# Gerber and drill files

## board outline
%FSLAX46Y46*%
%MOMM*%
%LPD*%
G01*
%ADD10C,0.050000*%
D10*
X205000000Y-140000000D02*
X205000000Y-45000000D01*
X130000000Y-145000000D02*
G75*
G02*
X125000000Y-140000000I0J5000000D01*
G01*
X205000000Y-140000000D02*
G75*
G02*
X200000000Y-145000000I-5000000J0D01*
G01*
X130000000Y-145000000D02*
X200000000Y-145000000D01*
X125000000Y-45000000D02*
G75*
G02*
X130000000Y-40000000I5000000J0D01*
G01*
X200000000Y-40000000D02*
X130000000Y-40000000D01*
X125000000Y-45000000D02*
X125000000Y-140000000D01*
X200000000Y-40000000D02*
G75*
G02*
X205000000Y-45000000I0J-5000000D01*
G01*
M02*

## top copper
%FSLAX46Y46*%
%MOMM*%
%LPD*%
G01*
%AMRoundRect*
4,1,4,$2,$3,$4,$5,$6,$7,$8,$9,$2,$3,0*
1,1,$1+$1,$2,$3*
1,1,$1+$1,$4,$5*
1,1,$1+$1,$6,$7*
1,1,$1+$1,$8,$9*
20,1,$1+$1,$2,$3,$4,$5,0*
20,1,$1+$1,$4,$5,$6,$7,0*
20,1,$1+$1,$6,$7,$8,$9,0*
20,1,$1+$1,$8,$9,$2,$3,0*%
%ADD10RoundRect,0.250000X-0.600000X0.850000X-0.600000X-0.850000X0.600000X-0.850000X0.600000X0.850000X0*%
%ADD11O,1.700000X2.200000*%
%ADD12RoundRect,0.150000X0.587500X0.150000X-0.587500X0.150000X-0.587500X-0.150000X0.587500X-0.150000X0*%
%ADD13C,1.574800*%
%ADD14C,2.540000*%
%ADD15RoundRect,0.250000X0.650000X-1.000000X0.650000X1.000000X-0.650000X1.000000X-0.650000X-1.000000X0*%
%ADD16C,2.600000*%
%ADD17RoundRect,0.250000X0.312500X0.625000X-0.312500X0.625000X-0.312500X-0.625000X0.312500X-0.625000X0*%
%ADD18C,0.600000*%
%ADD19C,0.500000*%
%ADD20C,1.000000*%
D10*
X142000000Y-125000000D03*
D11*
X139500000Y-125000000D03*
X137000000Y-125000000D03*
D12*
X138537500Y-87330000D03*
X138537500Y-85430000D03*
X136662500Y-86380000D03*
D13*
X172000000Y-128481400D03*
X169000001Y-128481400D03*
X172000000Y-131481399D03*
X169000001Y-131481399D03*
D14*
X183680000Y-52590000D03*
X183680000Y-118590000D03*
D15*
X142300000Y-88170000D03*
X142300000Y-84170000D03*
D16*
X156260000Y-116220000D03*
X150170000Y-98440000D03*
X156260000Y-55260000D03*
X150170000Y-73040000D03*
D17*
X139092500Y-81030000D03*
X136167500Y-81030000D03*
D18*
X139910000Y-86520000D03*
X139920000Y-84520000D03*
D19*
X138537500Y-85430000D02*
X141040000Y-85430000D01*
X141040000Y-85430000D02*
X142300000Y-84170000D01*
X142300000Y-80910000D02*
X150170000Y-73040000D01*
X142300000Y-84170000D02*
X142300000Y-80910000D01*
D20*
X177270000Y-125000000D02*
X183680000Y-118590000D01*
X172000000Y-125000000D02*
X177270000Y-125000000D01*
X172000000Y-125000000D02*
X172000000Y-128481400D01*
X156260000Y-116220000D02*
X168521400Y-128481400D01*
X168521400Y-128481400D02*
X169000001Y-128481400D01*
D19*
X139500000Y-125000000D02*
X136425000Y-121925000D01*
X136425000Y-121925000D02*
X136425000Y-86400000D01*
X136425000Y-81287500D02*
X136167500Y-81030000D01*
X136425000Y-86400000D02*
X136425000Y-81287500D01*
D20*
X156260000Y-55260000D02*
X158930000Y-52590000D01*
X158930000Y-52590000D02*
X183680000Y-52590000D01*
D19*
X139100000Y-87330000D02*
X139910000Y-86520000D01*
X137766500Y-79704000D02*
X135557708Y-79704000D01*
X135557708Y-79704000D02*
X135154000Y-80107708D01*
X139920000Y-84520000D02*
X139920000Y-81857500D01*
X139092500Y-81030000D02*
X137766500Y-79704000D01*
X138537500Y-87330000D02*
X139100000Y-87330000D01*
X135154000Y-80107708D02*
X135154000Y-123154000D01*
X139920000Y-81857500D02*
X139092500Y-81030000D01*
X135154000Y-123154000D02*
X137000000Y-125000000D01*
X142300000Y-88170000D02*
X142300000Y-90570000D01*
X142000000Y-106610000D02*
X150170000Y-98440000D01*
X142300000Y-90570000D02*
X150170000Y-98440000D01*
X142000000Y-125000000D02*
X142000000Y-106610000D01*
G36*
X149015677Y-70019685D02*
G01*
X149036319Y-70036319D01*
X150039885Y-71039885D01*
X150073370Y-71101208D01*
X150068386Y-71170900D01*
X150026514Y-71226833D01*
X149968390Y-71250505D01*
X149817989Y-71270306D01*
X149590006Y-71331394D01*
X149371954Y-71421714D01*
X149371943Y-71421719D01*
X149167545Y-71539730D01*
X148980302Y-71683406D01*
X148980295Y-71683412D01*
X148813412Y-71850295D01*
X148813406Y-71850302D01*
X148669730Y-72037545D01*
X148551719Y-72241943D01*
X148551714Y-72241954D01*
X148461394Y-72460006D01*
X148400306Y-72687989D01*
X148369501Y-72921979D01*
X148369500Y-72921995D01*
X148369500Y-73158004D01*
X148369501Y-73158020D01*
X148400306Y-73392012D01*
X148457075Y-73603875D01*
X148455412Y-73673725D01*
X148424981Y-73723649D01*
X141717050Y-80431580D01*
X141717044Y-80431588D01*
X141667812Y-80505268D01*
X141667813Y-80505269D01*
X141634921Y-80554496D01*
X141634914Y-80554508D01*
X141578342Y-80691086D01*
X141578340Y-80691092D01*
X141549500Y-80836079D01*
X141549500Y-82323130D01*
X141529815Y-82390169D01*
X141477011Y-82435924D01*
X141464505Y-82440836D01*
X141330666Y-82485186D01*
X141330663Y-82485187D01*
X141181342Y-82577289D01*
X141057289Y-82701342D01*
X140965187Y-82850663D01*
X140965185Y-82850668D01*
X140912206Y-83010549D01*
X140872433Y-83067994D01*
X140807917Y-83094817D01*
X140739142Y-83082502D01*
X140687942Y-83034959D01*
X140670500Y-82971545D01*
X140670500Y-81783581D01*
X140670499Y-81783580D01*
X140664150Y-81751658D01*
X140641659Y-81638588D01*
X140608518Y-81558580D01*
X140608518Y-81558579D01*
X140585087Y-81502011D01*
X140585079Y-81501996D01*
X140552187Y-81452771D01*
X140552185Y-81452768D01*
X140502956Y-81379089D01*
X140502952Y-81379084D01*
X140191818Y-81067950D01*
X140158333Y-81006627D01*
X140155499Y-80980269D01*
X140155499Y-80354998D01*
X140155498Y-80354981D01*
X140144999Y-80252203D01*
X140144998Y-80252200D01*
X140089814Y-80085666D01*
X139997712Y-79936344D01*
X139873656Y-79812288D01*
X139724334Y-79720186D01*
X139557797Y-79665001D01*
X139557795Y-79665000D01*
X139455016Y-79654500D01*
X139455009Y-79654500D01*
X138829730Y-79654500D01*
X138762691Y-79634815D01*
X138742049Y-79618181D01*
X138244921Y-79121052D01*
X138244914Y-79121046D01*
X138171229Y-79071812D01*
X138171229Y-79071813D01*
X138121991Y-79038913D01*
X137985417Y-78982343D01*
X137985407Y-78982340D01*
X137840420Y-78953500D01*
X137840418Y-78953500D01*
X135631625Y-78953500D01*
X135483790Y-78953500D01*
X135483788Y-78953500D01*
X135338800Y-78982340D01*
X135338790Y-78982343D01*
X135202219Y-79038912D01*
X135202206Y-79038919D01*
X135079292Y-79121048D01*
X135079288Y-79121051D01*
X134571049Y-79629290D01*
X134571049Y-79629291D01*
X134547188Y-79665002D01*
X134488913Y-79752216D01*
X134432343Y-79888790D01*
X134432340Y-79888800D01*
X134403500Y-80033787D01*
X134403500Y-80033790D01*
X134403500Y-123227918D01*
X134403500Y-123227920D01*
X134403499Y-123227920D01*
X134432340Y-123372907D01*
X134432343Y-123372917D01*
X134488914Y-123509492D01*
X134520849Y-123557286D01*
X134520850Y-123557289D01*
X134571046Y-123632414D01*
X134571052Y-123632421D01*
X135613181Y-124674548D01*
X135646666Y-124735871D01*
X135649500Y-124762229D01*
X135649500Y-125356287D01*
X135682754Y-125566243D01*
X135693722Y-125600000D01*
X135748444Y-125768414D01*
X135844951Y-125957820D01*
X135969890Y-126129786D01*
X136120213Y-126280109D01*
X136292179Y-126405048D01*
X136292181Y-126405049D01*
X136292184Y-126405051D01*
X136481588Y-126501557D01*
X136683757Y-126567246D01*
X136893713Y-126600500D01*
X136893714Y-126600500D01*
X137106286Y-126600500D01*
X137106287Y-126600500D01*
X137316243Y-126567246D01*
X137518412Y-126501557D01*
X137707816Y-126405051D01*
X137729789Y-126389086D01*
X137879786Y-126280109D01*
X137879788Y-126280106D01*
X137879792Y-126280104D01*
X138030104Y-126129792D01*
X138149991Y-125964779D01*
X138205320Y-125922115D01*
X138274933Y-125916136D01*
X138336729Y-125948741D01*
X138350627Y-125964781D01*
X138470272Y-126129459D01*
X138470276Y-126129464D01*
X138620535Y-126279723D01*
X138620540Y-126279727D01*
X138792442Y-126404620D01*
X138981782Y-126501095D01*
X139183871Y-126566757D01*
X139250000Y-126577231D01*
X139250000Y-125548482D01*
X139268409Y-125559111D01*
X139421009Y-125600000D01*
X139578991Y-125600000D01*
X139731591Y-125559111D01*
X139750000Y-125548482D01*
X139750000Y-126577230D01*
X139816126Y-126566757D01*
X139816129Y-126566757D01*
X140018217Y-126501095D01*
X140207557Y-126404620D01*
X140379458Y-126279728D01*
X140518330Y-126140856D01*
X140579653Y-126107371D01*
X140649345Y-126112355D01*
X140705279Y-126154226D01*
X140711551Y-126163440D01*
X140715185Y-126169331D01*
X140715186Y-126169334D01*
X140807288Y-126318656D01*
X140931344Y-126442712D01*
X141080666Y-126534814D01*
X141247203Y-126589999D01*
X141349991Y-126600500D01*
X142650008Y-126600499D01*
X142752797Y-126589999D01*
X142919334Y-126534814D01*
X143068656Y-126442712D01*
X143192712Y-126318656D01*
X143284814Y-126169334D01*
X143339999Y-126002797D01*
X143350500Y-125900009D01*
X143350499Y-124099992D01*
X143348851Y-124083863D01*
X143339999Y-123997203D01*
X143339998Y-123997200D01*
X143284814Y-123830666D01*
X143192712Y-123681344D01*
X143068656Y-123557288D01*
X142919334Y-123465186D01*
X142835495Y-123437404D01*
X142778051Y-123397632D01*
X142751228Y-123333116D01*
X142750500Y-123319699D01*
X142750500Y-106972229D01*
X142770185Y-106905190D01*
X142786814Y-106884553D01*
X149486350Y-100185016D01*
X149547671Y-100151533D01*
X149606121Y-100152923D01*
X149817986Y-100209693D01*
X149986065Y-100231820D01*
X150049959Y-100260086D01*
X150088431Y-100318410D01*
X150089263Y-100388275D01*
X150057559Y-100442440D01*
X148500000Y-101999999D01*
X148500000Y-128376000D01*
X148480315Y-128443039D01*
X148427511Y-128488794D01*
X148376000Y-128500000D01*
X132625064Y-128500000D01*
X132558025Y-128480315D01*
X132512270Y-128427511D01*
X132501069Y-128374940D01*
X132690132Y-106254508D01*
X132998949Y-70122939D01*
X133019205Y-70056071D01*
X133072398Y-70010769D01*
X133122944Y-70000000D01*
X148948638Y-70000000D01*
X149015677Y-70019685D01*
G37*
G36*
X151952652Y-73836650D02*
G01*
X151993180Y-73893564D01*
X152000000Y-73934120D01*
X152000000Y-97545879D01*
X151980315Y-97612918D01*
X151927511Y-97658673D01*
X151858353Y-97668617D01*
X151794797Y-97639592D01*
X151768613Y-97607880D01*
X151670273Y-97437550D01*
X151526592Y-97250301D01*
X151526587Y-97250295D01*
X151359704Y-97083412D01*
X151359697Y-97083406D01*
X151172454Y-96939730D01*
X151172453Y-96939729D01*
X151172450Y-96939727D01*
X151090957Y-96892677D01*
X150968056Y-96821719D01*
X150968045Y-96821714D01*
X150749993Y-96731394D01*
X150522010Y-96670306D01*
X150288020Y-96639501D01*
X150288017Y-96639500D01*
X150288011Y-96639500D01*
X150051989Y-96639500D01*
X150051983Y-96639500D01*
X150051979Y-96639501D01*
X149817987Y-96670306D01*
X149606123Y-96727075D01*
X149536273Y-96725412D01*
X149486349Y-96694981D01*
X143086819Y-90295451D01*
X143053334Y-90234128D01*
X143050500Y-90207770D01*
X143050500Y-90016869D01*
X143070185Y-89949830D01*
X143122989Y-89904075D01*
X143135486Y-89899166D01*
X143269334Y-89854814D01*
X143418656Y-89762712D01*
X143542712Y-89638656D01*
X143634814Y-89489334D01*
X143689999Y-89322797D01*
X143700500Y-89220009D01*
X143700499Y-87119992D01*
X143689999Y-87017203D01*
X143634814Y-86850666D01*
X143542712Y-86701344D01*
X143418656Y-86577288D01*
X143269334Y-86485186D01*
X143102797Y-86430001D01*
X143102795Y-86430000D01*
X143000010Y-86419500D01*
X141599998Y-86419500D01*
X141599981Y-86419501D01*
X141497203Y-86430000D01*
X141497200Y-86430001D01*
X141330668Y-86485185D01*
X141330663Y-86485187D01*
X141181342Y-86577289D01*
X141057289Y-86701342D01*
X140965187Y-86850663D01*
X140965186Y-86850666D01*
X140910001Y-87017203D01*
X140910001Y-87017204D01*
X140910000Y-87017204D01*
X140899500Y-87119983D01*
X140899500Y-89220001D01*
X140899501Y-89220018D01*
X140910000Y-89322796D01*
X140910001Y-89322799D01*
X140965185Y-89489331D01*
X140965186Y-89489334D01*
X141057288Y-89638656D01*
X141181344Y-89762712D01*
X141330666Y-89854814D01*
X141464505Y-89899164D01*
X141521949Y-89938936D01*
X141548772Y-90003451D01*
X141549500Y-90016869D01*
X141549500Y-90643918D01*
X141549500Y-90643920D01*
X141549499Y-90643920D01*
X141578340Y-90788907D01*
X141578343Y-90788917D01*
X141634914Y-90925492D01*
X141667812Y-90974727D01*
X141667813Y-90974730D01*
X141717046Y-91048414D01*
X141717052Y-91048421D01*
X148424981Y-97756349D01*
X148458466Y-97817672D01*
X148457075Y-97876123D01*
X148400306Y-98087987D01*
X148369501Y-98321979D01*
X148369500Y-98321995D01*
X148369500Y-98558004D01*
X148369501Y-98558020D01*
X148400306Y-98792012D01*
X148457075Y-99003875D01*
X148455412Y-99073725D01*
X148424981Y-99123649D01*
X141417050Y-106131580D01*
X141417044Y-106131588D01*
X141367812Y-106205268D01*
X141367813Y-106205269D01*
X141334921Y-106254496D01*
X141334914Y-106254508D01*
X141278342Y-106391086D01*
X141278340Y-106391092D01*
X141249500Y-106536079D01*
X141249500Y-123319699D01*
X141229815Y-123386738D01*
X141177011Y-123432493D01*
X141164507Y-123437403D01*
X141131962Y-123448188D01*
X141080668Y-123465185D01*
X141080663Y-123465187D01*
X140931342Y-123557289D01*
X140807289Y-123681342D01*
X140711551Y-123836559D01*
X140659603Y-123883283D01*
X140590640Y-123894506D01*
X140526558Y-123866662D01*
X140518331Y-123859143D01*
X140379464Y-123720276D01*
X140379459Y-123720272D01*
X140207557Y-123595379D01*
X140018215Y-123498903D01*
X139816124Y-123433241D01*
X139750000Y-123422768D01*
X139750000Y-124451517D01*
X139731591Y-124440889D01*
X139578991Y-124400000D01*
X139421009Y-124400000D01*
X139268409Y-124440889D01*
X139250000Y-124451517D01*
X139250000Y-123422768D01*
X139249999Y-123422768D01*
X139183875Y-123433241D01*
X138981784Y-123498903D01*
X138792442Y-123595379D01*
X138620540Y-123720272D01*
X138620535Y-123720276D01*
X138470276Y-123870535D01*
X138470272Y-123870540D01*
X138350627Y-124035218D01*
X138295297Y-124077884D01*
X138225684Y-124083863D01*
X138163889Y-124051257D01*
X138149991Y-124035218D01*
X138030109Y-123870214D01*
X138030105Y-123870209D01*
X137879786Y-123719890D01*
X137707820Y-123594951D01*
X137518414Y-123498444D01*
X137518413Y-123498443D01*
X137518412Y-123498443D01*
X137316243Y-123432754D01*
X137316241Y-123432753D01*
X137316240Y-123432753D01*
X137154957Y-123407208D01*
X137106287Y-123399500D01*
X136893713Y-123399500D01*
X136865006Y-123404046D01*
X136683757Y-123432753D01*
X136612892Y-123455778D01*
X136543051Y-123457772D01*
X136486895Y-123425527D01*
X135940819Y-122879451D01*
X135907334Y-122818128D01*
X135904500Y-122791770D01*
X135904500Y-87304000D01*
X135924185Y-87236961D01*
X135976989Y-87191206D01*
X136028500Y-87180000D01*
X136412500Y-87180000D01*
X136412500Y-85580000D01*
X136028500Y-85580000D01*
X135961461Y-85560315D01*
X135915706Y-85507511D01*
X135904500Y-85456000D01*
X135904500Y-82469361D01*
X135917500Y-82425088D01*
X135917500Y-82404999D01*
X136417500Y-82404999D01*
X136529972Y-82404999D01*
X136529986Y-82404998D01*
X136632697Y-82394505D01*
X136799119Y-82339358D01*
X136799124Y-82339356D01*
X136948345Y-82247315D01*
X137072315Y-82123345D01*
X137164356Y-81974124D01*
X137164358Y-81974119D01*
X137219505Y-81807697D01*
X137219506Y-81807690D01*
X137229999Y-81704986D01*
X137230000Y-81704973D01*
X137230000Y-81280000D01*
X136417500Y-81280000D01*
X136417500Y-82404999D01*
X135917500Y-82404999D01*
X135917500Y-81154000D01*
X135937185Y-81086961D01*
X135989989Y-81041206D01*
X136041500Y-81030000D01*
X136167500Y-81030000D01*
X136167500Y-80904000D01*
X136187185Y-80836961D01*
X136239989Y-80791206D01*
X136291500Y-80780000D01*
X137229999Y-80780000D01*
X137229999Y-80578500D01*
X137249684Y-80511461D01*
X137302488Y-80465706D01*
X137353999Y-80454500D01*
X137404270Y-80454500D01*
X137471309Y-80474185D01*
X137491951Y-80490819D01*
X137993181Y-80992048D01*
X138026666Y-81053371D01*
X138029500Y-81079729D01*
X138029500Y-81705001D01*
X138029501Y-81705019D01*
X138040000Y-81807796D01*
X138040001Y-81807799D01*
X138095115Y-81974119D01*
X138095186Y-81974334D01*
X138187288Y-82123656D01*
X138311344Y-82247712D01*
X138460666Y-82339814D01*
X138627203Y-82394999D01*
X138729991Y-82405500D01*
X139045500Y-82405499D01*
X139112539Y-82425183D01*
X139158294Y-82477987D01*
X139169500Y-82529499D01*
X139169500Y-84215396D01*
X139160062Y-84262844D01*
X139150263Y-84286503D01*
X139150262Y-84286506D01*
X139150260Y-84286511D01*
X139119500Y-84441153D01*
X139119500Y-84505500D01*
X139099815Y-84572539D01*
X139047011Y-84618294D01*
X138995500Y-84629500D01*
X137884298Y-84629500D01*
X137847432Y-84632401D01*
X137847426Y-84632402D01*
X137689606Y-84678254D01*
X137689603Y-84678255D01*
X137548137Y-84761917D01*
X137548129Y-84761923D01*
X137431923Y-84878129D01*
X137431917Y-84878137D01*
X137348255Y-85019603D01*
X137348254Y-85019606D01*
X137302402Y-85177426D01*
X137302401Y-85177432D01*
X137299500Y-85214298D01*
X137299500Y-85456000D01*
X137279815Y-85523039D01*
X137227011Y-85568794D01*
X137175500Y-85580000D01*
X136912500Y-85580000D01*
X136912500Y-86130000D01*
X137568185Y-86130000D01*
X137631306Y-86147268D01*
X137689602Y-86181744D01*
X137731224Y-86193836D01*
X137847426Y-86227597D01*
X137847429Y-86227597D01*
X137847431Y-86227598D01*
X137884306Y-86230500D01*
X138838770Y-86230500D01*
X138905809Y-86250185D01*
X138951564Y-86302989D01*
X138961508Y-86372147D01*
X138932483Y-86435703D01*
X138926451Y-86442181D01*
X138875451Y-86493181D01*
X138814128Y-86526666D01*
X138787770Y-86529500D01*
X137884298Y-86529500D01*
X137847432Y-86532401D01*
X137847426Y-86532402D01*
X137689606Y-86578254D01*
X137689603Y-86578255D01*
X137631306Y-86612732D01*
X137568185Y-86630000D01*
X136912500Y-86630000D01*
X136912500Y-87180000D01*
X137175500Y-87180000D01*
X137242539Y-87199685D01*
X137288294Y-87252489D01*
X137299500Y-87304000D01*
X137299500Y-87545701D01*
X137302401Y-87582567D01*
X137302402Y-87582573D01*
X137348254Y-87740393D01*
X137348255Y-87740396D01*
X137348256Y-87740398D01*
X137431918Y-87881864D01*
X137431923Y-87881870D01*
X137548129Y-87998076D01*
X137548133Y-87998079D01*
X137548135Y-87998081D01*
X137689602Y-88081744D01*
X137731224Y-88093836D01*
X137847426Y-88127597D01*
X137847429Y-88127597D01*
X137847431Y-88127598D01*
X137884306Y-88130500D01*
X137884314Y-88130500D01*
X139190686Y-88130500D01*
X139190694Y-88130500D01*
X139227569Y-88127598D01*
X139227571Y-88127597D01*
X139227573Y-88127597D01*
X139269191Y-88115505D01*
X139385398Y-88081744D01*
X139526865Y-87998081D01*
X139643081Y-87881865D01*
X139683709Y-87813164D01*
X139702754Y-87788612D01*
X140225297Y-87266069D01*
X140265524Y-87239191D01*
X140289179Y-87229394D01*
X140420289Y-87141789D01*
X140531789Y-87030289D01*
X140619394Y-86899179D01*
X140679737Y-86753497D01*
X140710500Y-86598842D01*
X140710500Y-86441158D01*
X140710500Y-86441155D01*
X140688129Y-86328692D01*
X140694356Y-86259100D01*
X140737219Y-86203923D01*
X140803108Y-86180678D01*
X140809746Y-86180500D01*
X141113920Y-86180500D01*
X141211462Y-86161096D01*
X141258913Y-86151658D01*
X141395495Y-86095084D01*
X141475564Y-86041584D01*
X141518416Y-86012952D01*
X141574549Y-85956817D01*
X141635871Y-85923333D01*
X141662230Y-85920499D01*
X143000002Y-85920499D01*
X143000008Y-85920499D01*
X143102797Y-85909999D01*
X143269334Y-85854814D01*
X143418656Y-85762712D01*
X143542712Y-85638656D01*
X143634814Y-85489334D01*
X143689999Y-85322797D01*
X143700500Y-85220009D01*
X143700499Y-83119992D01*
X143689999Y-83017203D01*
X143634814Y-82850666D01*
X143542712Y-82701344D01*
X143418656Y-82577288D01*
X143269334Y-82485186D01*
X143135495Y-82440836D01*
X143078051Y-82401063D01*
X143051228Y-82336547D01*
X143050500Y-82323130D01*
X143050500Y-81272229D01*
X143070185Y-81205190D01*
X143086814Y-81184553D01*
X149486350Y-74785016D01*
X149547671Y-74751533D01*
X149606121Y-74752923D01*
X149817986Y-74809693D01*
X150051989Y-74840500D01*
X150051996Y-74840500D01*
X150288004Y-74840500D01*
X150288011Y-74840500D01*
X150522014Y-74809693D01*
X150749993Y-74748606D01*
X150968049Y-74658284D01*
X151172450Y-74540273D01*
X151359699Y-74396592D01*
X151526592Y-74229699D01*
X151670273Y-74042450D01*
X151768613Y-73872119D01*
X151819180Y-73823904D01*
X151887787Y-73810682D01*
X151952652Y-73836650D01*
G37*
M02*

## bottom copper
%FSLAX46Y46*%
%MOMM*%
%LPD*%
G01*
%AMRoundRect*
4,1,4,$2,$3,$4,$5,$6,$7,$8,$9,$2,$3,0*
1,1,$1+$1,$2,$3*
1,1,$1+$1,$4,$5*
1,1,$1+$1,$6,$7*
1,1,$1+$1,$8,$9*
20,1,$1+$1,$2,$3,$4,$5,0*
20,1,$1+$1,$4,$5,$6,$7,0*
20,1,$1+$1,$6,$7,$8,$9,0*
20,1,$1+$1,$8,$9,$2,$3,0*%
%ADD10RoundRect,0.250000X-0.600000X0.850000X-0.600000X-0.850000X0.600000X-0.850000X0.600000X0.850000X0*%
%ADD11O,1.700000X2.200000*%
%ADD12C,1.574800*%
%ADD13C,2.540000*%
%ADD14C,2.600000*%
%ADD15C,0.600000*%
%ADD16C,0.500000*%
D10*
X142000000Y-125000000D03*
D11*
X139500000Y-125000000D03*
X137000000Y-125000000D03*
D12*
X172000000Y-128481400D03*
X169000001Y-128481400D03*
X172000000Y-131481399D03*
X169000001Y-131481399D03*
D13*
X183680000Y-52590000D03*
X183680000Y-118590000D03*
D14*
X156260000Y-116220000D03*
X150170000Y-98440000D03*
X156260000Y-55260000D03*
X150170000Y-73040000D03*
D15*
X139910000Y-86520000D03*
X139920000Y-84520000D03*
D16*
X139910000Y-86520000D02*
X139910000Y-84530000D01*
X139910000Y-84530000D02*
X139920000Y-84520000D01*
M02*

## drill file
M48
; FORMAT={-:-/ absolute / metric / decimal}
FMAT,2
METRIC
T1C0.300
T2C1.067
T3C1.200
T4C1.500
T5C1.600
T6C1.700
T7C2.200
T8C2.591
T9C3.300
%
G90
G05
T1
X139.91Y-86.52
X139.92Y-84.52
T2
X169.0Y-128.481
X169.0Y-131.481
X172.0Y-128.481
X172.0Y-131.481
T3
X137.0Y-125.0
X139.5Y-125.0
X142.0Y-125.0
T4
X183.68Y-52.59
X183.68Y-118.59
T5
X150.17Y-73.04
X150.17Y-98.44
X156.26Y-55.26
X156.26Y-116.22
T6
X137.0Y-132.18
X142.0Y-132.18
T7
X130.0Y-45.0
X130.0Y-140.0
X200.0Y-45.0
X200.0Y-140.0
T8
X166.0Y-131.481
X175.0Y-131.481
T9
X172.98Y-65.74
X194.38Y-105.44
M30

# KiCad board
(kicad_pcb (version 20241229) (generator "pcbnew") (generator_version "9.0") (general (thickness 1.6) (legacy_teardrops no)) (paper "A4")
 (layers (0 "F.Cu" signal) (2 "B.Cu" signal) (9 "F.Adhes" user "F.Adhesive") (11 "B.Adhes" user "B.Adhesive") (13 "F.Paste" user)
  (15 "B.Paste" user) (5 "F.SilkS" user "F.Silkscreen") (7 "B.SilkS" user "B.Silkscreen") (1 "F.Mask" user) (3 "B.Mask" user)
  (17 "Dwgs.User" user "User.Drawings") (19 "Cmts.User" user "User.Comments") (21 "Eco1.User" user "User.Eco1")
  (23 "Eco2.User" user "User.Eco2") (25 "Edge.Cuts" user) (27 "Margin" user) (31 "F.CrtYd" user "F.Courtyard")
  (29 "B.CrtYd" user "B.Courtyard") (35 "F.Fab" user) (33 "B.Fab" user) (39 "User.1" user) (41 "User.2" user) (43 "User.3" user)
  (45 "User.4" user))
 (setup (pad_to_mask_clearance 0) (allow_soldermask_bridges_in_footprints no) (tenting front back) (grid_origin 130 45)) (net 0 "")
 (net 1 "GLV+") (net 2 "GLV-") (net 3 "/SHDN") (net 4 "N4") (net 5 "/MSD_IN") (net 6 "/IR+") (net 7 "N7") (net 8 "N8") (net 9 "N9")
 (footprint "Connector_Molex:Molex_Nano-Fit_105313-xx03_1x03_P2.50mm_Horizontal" (layer "F.Cu") (at 142 125 -90)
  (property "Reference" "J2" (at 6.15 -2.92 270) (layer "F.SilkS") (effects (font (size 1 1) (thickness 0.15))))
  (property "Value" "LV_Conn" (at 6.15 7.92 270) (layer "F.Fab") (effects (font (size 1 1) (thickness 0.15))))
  (pad "" np_thru_hole circle (at 7.18 0 270) (size 1.7 1.7) (drill 1.7) (layers "*.Cu" "*.Mask"))
  (pad "" np_thru_hole circle (at 7.18 5 270) (size 1.7 1.7) (drill 1.7) (layers "*.Cu" "*.Mask"))
  (pad "1" thru_hole roundrect (at 0 0 270) (size 2.2 1.7) (drill 1.2) (layers "*.Cu" "*.Mask") (remove_unused_layers no)
   (roundrect_rratio 0.147059) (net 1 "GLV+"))
  (pad "2" thru_hole oval (at 0 2.5 270) (size 2.2 1.7) (drill 1.2) (layers "*.Cu" "*.Mask") (remove_unused_layers no) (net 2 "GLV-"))
  (pad "3" thru_hole oval (at 0 5 270) (size 2.2 1.7) (drill 1.2) (layers "*.Cu" "*.Mask") (remove_unused_layers no) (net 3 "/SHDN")))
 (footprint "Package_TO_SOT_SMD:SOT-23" (layer "F.Cu") (at 137.6 86.38 180)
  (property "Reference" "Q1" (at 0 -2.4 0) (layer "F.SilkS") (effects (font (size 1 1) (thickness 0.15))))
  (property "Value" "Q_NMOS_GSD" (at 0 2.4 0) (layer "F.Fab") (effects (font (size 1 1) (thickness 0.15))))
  (pad "1" smd roundrect (at -0.9375 -0.95 180) (size 1.475 0.6) (layers "F.Cu" "F.Mask" "F.Paste") (roundrect_rratio 0.25) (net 3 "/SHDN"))
  (pad "2" smd roundrect (at -0.9375 0.95 180) (size 1.475 0.6) (layers "F.Cu" "F.Mask" "F.Paste") (roundrect_rratio 0.25) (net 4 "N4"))
  (pad "3" smd roundrect (at 0.9375 0 180) (size 1.475 0.6) (layers "F.Cu" "F.Mask" "F.Paste") (roundrect_rratio 0.25) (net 2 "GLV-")))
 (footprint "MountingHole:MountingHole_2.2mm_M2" (layer "F.Cu") (at 200 45)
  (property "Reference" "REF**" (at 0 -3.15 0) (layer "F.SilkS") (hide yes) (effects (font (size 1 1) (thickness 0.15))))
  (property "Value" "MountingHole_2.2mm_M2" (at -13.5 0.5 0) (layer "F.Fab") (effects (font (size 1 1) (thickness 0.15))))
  (pad "" np_thru_hole circle (at 0 0) (size 2.2 2.2) (drill 2.2) (layers "*.Cu" "*.Mask")))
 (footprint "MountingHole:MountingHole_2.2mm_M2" (layer "F.Cu") (at 130 140)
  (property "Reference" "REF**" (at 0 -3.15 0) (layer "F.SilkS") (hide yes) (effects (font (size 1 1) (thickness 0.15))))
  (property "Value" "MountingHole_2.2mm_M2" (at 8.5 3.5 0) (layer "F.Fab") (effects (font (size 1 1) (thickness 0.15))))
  (pad "" np_thru_hole circle (at 0 0) (size 2.2 2.2) (drill 2.2) (layers "*.Cu" "*.Mask")))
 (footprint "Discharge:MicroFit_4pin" (layer "F.Cu") (at 170.7484 130 180)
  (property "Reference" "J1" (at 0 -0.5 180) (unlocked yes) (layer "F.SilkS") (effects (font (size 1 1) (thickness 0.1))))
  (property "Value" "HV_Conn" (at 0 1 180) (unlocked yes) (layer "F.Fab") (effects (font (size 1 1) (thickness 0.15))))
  (pad "" np_thru_hole circle (at -4.251599 -1.481399 180) (size 2.5908 2.5908) (drill 2.5908) (layers))
  (pad "" np_thru_hole circle (at 4.748398 -1.481399 180) (size 2.5908 2.5908) (drill 2.5908) (layers))
  (pad "1" thru_hole circle (at -1.2516 1.5186 180) (size 1.5748 1.5748) (drill 1.0668) (layers "*.Cu" "*.Mask") (remove_unused_layers no)
   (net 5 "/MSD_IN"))
  (pad "2" thru_hole circle (at 1.748399 1.5186 180) (size 1.5748 1.5748) (drill 1.0668) (layers "*.Cu" "*.Mask") (remove_unused_layers no)
   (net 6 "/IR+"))
  (pad "3" thru_hole circle (at -1.2516 -1.481399 180) (size 1.5748 1.5748) (drill 1.0668) (layers "*.Cu" "*.Mask")
   (remove_unused_layers no) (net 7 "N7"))
  (pad "4" thru_hole circle (at 1.748399 -1.481399 180) (size 1.5748 1.5748) (drill 1.0668) (layers "*.Cu" "*.Mask")
   (remove_unused_layers no) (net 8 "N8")))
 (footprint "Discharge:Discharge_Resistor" (layer "F.Cu") (at 183.68 85.59 -90)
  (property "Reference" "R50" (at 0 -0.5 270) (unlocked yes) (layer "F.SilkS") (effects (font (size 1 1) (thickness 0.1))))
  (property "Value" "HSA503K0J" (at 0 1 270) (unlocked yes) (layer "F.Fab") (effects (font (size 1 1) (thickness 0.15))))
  (pad "" np_thru_hole circle (at -19.85 10.7 270) (size 3.3 3.3) (drill 3.3) (layers "*.Cu" "*.Mask"))
  (pad "" np_thru_hole circle (at 19.85 -10.7 270) (size 3.3 3.3) (drill 3.3) (layers "*.Cu" "*.Mask"))
  (pad "1" thru_hole circle (at -33 0 270) (size 2.54 2.54) (drill 1.5) (layers "*.Cu" "*.Mask") (remove_unused_layers no) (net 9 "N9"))
  (pad "2" thru_hole circle (at 33 0 270) (size 2.54 2.54) (drill 1.5) (layers "*.Cu" "*.Mask") (remove_unused_layers no) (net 5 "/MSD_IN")))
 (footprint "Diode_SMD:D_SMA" (layer "F.Cu") (at 142.3 86.17 90)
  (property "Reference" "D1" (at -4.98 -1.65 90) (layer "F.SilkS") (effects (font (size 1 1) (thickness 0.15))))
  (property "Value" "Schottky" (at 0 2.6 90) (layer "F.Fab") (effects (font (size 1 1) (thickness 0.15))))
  (pad "1" smd roundrect (at -2 0 90) (size 2.5 1.8) (layers "F.Cu" "F.Mask" "F.Paste") (roundrect_rratio 0.1388888889) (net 1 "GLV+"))
  (pad "2" smd roundrect (at 2 0 90) (size 2.5 1.8) (layers "F.Cu" "F.Mask" "F.Paste") (roundrect_rratio 0.1388888889) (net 4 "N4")))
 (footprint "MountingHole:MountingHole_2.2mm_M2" (layer "F.Cu") (at 130 45)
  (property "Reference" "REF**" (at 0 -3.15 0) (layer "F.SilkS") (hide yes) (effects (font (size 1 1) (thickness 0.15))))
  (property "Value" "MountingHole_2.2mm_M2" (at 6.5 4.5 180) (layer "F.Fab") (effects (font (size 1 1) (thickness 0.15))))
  (pad "" np_thru_hole circle (at 0 0) (size 2.2 2.2) (drill 2.2) (layers "*.Cu" "*.Mask")))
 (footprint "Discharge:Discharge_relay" (layer "F.Cu") (at 154.555 85.74 -90)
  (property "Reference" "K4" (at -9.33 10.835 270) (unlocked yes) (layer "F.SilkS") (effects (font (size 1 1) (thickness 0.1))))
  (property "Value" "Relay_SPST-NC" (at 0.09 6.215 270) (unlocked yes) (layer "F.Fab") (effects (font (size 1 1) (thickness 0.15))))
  (pad "1" thru_hole circle (at 30.48 -1.705 90) (size 2.6 2.6) (drill 1.6) (layers "*.Cu" "*.Mask") (remove_unused_layers no)
   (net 6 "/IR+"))
  (pad "2" thru_hole circle (at 12.7 4.385 90) (size 2.6 2.6) (drill 1.6) (layers "*.Cu" "*.Mask") (remove_unused_layers no) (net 1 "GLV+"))
  (pad "4" thru_hole circle (at -30.48 -1.705 90) (size 2.6 2.6) (drill 1.6) (layers "*.Cu" "*.Mask") (remove_unused_layers no) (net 9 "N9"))
  (pad "5" thru_hole circle (at -12.7 4.385 90) (size 2.6 2.6) (drill 1.6) (layers "*.Cu" "*.Mask") (remove_unused_layers no) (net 4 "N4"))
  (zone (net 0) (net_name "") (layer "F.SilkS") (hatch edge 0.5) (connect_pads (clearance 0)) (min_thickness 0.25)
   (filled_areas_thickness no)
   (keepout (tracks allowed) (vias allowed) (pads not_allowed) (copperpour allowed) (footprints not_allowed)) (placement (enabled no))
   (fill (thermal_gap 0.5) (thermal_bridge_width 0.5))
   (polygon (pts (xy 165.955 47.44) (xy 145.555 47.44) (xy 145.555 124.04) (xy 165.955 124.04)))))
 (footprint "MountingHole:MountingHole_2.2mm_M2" (layer "F.Cu") (at 200 140)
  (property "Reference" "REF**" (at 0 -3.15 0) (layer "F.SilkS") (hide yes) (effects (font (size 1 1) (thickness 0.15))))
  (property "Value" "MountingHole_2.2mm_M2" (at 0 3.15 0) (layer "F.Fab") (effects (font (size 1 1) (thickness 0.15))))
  (pad "" np_thru_hole circle (at 0 0) (size 2.2 2.2) (drill 2.2) (layers "*.Cu" "*.Mask")))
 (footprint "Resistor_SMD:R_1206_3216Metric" (layer "F.Cu") (at 137.63 81.03 180)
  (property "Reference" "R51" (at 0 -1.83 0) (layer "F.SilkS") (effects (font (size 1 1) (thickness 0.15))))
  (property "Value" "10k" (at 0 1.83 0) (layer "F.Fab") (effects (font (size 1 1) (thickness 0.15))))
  (pad "1" smd roundrect (at -1.4625 0 180) (size 1.125 1.75) (layers "F.Cu" "F.Mask" "F.Paste") (roundrect_rratio 0.222222) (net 3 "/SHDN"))
  (pad "2" smd roundrect (at 1.4625 0 180) (size 1.125 1.75) (layers "F.Cu" "F.Mask" "F.Paste") (roundrect_rratio 0.222222) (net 2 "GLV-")))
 (gr_line (start 205 140) (end 205 45) (stroke (width 0.05) (type default)) (layer "Edge.Cuts"))
 (gr_arc (start 130 145) (mid 126.464466 143.535534) (end 125 140) (stroke (width 0.05) (type default)) (layer "Edge.Cuts"))
 (gr_arc (start 205 140) (mid 203.535534 143.535534) (end 200 145) (stroke (width 0.05) (type default)) (layer "Edge.Cuts"))
 (gr_line (start 130 145) (end 200 145) (stroke (width 0.05) (type default)) (layer "Edge.Cuts"))
 (gr_arc (start 125 45) (mid 126.464466 41.464466) (end 130 40) (stroke (width 0.05) (type default)) (layer "Edge.Cuts"))
 (gr_line (start 200 40) (end 130 40) (stroke (width 0.05) (type default)) (layer "Edge.Cuts"))
 (gr_line (start 125 45) (end 125 140) (stroke (width 0.05) (type default)) (layer "Edge.Cuts"))
 (gr_arc (start 200 40) (mid 203.535534 41.464466) (end 205 45) (stroke (width 0.05) (type default)) (layer "Edge.Cuts"))
 (segment (start 138.5375 85.43) (end 141.04 85.43) (width 0.5) (layer "F.Cu") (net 4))
 (segment (start 141.04 85.43) (end 142.3 84.17) (width 0.5) (layer "F.Cu") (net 4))
 (segment (start 142.3 80.91) (end 150.17 73.04) (width 0.5) (layer "F.Cu") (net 4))
 (segment (start 142.3 84.17) (end 142.3 80.91) (width 0.5) (layer "F.Cu") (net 4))
 (segment (start 177.27 125) (end 183.68 118.59) (width 1) (layer "F.Cu") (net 5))
 (segment (start 172 125) (end 177.27 125) (width 1) (layer "F.Cu") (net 5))
 (segment (start 172 125) (end 172 128.4814) (width 1) (layer "F.Cu") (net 5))
 (segment (start 156.26 116.22) (end 168.5214 128.4814) (width 1) (layer "F.Cu") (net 6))
 (segment (start 168.5214 128.4814) (end 169.000001 128.4814) (width 1) (layer "F.Cu") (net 6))
 (segment (start 139.5 125) (end 136.425 121.925) (width 0.5) (layer "F.Cu") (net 2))
 (segment (start 136.425 121.925) (end 136.425 86.4) (width 0.5) (layer "F.Cu") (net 2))
 (segment (start 136.425 81.2875) (end 136.1675 81.03) (width 0.5) (layer "F.Cu") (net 2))
 (segment (start 136.425 86.4) (end 136.425 81.2875) (width 0.5) (layer "F.Cu") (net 2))
 (segment (start 156.26 55.26) (end 158.93 52.59) (width 1) (layer "F.Cu") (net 9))
 (segment (start 158.93 52.59) (end 183.68 52.59) (width 1) (layer "F.Cu") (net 9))
 (segment (start 139.1 87.33) (end 139.91 86.52) (width 0.5) (layer "F.Cu") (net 3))
 (segment (start 137.7665 79.704) (end 135.557708 79.704) (width 0.5) (layer "F.Cu") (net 3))
 (segment (start 135.557708 79.704) (end 135.154 80.107708) (width 0.5) (layer "F.Cu") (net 3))
 (segment (start 139.92 84.52) (end 139.92 81.8575) (width 0.5) (layer "F.Cu") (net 3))
 (segment (start 139.0925 81.03) (end 137.7665 79.704) (width 0.5) (layer "F.Cu") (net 3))
 (segment (start 138.5375 87.33) (end 139.1 87.33) (width 0.5) (layer "F.Cu") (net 3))
 (segment (start 135.154 80.107708) (end 135.154 123.154) (width 0.5) (layer "F.Cu") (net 3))
 (segment (start 139.92 81.8575) (end 139.0925 81.03) (width 0.5) (layer "F.Cu") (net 3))
 (segment (start 135.154 123.154) (end 137 125) (width 0.5) (layer "F.Cu") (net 3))
 (via (at 139.91 86.52) (size 0.6) (drill 0.3) (layers "F.Cu" "B.Cu") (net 3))
 (via (at 139.92 84.52) (size 0.6) (drill 0.3) (layers "F.Cu" "B.Cu") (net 3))
 (segment (start 139.91 86.52) (end 139.91 84.53) (width 0.5) (layer "B.Cu") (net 3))
 (segment (start 139.91 84.53) (end 139.92 84.52) (width 0.5) (layer "B.Cu") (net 3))
 (segment (start 142.3 88.17) (end 142.3 90.57) (width 0.5) (layer "F.Cu") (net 1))
 (segment (start 142 106.61) (end 150.17 98.44) (width 0.5) (layer "F.Cu") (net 1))
 (segment (start 142.3 90.57) (end 150.17 98.44) (width 0.5) (layer "F.Cu") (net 1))
 (segment (start 142 125) (end 142 106.61) (width 0.5) (layer "F.Cu") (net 1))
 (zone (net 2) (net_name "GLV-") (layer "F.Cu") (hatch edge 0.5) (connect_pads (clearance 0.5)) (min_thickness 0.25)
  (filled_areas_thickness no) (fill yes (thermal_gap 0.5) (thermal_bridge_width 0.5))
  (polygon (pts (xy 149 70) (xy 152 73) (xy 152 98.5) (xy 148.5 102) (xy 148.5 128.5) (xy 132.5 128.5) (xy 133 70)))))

